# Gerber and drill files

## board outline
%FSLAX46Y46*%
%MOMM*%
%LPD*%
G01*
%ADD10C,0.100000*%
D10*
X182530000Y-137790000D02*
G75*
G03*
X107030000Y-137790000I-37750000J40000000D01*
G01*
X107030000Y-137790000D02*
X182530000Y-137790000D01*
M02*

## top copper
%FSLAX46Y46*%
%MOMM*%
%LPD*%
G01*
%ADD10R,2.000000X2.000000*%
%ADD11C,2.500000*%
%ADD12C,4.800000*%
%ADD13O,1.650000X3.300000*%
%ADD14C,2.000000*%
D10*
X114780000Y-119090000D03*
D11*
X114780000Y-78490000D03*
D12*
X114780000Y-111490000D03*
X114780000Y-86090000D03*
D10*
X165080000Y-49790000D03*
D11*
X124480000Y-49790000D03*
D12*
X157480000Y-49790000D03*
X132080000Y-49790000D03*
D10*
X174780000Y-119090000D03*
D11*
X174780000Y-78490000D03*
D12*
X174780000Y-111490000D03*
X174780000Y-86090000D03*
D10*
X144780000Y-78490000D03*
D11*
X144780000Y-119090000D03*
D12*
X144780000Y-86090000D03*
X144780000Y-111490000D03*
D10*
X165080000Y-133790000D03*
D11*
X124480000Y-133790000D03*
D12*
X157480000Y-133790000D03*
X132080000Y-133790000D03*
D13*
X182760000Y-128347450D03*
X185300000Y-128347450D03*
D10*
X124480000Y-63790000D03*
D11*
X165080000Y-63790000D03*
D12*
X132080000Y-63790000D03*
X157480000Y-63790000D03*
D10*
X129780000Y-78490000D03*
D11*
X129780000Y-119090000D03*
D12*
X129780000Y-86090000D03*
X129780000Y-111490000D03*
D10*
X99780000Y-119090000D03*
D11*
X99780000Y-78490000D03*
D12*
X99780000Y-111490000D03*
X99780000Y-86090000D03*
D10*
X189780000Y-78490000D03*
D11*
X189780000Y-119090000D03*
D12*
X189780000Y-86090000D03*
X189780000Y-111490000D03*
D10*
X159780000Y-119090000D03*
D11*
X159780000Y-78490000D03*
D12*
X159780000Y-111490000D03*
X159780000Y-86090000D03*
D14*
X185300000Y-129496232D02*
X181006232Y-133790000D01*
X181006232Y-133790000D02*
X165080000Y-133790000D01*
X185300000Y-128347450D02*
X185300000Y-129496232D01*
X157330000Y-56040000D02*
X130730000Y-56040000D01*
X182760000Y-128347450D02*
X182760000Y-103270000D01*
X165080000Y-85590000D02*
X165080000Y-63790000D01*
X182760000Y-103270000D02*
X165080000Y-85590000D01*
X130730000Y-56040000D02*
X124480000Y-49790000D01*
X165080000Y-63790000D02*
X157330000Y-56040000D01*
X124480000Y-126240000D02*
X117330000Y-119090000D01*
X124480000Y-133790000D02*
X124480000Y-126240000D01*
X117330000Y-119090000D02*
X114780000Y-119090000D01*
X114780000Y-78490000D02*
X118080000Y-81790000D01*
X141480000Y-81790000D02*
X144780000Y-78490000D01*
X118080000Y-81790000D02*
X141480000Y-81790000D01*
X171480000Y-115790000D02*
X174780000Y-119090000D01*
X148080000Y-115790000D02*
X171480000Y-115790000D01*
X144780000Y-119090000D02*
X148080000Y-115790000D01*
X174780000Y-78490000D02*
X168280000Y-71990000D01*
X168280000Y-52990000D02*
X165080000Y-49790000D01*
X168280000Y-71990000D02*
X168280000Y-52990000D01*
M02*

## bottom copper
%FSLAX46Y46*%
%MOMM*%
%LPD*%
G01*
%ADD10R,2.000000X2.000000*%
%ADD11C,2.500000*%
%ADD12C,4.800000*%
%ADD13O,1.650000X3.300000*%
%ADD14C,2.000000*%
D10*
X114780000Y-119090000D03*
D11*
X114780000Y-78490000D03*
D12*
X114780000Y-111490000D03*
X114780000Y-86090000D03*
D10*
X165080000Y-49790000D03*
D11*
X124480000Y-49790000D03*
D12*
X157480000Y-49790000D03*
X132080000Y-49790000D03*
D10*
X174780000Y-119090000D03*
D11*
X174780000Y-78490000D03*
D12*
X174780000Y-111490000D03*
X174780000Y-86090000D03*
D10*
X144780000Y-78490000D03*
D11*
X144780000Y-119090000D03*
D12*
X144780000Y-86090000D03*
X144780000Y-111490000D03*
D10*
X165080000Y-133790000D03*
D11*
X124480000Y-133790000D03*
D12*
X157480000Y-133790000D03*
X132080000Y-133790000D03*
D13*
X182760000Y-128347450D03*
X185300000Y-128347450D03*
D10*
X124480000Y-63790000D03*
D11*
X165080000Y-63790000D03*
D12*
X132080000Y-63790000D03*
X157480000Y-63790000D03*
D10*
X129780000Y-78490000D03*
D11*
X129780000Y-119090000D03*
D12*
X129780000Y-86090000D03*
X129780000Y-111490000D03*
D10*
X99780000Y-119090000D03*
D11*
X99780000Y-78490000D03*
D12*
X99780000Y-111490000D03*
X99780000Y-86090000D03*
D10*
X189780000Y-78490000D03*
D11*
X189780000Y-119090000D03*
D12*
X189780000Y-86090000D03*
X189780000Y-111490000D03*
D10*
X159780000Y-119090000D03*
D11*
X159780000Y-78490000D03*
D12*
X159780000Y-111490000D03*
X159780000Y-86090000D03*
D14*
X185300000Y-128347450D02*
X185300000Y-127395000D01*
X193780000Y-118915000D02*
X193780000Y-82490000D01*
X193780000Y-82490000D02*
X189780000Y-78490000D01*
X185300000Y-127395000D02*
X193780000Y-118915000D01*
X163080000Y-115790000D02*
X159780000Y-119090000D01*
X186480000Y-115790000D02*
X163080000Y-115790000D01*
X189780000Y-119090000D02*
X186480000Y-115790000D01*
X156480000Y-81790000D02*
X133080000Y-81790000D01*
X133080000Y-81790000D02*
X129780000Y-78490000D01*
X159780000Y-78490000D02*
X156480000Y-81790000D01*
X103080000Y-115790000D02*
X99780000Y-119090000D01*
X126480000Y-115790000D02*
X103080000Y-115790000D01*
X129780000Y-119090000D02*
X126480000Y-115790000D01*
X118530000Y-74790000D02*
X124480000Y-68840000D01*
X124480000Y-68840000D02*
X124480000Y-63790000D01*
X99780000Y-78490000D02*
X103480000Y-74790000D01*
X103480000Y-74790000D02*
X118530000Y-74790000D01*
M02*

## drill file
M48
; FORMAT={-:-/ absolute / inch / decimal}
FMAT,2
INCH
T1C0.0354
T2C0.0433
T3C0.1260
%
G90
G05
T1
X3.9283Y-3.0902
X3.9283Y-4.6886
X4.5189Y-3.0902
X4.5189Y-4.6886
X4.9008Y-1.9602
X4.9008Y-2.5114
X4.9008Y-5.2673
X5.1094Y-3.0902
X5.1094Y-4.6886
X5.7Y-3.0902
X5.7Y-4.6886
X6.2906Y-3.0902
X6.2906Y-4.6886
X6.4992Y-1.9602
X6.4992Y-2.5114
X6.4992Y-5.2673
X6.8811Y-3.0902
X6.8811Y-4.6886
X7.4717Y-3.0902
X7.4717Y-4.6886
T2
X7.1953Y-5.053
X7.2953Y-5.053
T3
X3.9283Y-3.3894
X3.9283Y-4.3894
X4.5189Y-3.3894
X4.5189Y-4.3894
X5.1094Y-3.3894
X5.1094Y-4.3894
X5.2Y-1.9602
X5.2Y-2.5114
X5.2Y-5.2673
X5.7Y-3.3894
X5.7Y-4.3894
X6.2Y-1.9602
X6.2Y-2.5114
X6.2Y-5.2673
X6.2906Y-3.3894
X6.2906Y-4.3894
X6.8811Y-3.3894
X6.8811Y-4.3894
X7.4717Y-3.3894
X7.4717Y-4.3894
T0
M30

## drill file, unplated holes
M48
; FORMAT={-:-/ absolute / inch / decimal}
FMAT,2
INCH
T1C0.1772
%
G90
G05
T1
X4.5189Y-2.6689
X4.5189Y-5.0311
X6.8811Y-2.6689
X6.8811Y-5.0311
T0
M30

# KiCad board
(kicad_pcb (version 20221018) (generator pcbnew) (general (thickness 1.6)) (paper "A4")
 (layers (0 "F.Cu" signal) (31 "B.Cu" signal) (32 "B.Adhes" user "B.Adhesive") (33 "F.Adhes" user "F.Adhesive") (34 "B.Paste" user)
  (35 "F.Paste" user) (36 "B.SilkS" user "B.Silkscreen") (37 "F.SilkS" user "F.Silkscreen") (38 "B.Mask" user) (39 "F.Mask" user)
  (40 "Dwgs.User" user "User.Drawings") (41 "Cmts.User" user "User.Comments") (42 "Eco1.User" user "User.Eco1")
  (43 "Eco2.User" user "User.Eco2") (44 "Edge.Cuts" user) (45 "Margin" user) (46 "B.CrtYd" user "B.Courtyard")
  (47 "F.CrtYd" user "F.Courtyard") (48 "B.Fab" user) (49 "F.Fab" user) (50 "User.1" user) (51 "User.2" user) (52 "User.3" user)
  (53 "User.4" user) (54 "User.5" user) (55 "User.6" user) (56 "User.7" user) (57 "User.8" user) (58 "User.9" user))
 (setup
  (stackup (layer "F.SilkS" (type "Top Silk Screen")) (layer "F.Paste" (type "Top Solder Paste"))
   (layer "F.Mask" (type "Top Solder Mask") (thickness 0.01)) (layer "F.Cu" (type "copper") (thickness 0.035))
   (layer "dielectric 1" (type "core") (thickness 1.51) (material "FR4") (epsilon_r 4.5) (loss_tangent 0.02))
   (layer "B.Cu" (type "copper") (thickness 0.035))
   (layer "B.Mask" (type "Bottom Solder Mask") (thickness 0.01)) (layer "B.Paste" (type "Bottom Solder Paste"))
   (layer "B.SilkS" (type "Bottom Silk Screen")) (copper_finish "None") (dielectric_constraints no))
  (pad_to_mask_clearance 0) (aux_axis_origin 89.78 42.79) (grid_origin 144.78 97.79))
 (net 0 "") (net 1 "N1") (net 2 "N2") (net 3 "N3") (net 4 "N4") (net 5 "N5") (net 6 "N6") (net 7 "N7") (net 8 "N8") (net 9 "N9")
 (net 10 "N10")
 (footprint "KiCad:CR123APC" (layer "F.Cu") (at 114.78 119.09 90)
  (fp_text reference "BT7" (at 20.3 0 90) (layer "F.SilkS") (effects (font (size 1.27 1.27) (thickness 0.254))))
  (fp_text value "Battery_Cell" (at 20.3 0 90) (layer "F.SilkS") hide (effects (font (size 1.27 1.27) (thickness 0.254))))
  (pad "1" thru_hole rect (at 0 0 90) (size 2 2) (drill 0.9) (layers "*.Cu" "*.Mask") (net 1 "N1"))
  (pad "2" thru_hole circle (at 40.6 0 90) (size 2.5 2.5) (drill 0.9) (layers "*.Cu" "*.Mask") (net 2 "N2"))
  (pad "MH1" thru_hole circle (at 7.6 0 90) (size 4.8 4.8) (drill 3.2) (layers "*.Cu" "*.Mask"))
  (pad "MH2" thru_hole circle (at 33 0 90) (size 4.8 4.8) (drill 3.2) (layers "*.Cu" "*.Mask")))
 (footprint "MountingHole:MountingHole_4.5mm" (layer "F.Cu") (at 174.78 127.79)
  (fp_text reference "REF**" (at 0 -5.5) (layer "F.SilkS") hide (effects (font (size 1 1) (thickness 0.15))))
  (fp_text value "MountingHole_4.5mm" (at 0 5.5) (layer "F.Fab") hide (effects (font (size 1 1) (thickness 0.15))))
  (pad "" np_thru_hole circle (at 0 0) (size 4.5 4.5) (drill 4.5) (layers "*.Cu" "*.Mask")))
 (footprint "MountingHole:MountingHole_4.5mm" (layer "F.Cu") (at 174.78 67.79)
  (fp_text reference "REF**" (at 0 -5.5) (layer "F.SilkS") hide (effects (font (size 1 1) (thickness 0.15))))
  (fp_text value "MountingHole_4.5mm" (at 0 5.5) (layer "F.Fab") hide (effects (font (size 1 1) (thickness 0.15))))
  (pad "" np_thru_hole circle (at 0 0) (size 4.5 4.5) (drill 4.5) (layers "*.Cu" "*.Mask")))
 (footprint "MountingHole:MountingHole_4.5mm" (layer "F.Cu") (at 114.78 67.79)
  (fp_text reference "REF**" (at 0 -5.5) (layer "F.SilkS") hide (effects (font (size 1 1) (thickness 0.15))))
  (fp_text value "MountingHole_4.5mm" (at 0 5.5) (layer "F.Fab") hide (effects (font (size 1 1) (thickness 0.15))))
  (pad "" np_thru_hole circle (at 0 0) (size 4.5 4.5) (drill 4.5) (layers "*.Cu" "*.Mask")))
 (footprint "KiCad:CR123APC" (layer "F.Cu") (at 165.08 49.79 180)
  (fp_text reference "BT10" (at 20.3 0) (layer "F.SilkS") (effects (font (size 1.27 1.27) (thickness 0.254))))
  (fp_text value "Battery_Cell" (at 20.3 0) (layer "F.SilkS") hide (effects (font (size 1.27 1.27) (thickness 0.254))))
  (pad "1" thru_hole rect (at 0 0 180) (size 2 2) (drill 0.9) (layers "*.Cu" "*.Mask") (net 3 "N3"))
  (pad "2" thru_hole circle (at 40.6 0 180) (size 2.5 2.5) (drill 0.9) (layers "*.Cu" "*.Mask") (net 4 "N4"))
  (pad "MH1" thru_hole circle (at 7.6 0 180) (size 4.8 4.8) (drill 3.2) (layers "*.Cu" "*.Mask"))
  (pad "MH2" thru_hole circle (at 33 0 180) (size 4.8 4.8) (drill 3.2) (layers "*.Cu" "*.Mask")))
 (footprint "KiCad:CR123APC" (layer "F.Cu") (at 174.78 119.09 90)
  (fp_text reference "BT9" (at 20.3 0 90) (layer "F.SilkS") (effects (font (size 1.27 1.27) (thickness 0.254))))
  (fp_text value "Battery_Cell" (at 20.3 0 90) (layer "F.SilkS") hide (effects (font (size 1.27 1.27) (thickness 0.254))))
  (pad "1" thru_hole rect (at 0 0 90) (size 2 2) (drill 0.9) (layers "*.Cu" "*.Mask") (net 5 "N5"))
  (pad "2" thru_hole circle (at 40.6 0 90) (size 2.5 2.5) (drill 0.9) (layers "*.Cu" "*.Mask") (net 3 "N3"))
  (pad "MH1" thru_hole circle (at 7.6 0 90) (size 4.8 4.8) (drill 3.2) (layers "*.Cu" "*.Mask"))
  (pad "MH2" thru_hole circle (at 33 0 90) (size 4.8 4.8) (drill 3.2) (layers "*.Cu" "*.Mask")))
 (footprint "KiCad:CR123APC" (layer "F.Cu") (at 144.78 78.49 -90)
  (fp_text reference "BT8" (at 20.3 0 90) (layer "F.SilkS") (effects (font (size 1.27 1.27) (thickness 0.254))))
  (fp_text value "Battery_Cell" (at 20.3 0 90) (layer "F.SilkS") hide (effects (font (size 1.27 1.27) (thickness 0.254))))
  (pad "1" thru_hole rect (at 0 0 270) (size 2 2) (drill 0.9) (layers "*.Cu" "*.Mask") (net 2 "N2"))
  (pad "2" thru_hole circle (at 40.6 0 270) (size 2.5 2.5) (drill 0.9) (layers "*.Cu" "*.Mask") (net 5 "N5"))
  (pad "MH1" thru_hole circle (at 7.6 0 270) (size 4.8 4.8) (drill 3.2) (layers "*.Cu" "*.Mask"))
  (pad "MH2" thru_hole circle (at 33 0 270) (size 4.8 4.8) (drill 3.2) (layers "*.Cu" "*.Mask")))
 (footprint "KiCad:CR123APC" (layer "F.Cu") (at 165.08 133.79 180)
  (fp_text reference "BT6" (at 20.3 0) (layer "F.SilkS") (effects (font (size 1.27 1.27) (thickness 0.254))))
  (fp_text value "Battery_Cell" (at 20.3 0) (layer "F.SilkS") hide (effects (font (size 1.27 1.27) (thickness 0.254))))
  (pad "1" thru_hole rect (at 0 0 180) (size 2 2) (drill 0.9) (layers "*.Cu" "*.Mask") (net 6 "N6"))
  (pad "2" thru_hole circle (at 40.6 0 180) (size 2.5 2.5) (drill 0.9) (layers "*.Cu" "*.Mask") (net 1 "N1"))
  (pad "MH1" thru_hole circle (at 7.6 0 180) (size 4.8 4.8) (drill 3.2) (layers "*.Cu" "*.Mask"))
  (pad "MH2" thru_hole circle (at 33 0 180) (size 4.8 4.8) (drill 3.2) (layers "*.Cu" "*.Mask")))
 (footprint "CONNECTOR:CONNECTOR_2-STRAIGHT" (layer "F.Cu") (at 184.03 128.34745)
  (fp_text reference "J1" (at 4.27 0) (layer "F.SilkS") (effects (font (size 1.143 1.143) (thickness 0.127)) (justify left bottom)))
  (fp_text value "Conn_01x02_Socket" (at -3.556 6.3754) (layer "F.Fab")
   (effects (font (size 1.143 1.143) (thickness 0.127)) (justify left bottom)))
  (pad "1" thru_hole oval (at -1.27 0 90) (size 3.3 1.65) (drill 1.1) (layers "*.Cu" "*.Mask") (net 4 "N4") (solder_mask_margin 0.1016)
   (thermal_bridge_angle 45))
  (pad "2" thru_hole oval (at 1.27 0 90) (size 3.3 1.65) (drill 1.1) (layers "*.Cu" "*.Mask") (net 6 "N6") (solder_mask_margin 0.1016)
   (thermal_bridge_angle 45)))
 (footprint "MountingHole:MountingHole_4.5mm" (layer "F.Cu") (at 114.78 127.79)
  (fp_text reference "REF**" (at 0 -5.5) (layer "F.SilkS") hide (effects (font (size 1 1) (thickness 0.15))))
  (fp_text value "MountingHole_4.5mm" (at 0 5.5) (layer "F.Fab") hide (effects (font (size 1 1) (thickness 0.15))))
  (pad "" np_thru_hole circle (at 0 0) (size 4.5 4.5) (drill 4.5) (layers "*.Cu" "*.Mask")))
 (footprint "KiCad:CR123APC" (layer "B.Cu") (at 124.48 63.79)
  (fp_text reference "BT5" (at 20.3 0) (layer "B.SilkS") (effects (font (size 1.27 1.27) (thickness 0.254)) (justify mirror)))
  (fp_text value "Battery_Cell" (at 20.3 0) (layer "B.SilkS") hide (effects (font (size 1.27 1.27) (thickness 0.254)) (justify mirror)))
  (pad "1" thru_hole rect (at 0 0) (size 2 2) (drill 0.9) (layers "*.Cu" "*.Mask") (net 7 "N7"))
  (pad "2" thru_hole circle (at 40.6 0) (size 2.5 2.5) (drill 0.9) (layers "*.Cu" "*.Mask") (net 4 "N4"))
  (pad "MH1" thru_hole circle (at 7.6 0) (size 4.8 4.8) (drill 3.2) (layers "*.Cu" "*.Mask"))
  (pad "MH2" thru_hole circle (at 33 0) (size 4.8 4.8) (drill 3.2) (layers "*.Cu" "*.Mask")))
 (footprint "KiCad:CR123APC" (layer "B.Cu") (at 129.78 78.49 -90)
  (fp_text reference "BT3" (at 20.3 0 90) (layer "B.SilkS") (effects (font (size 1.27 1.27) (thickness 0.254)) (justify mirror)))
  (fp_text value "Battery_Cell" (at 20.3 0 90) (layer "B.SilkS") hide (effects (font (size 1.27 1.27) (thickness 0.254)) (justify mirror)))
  (pad "1" thru_hole rect (at 0 0 270) (size 2 2) (drill 0.9) (layers "*.Cu" "*.Mask") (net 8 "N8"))
  (pad "2" thru_hole circle (at 40.6 0 270) (size 2.5 2.5) (drill 0.9) (layers "*.Cu" "*.Mask") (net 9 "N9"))
  (pad "MH1" thru_hole circle (at 7.6 0 270) (size 4.8 4.8) (drill 3.2) (layers "*.Cu" "*.Mask"))
  (pad "MH2" thru_hole circle (at 33 0 270) (size 4.8 4.8) (drill 3.2) (layers "*.Cu" "*.Mask")))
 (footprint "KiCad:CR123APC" (layer "B.Cu") (at 99.78 119.09 90)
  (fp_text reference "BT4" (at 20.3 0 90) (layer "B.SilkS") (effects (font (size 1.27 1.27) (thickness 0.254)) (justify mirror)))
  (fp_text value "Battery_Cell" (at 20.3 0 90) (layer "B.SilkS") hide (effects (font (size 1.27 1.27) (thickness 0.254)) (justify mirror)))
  (pad "1" thru_hole rect (at 0 0 90) (size 2 2) (drill 0.9) (layers "*.Cu" "*.Mask") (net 9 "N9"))
  (pad "2" thru_hole circle (at 40.6 0 90) (size 2.5 2.5) (drill 0.9) (layers "*.Cu" "*.Mask") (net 7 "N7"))
  (pad "MH1" thru_hole circle (at 7.6 0 90) (size 4.8 4.8) (drill 3.2) (layers "*.Cu" "*.Mask"))
  (pad "MH2" thru_hole circle (at 33 0 90) (size 4.8 4.8) (drill 3.2) (layers "*.Cu" "*.Mask")))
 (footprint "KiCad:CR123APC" (layer "B.Cu") (at 189.78 78.49 -90)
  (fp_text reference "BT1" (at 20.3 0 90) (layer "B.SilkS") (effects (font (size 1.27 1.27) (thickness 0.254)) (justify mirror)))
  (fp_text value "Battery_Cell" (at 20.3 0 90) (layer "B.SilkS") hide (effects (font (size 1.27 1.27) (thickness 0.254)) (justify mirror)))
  (pad "1" thru_hole rect (at 0 0 270) (size 2 2) (drill 0.9) (layers "*.Cu" "*.Mask") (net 6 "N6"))
  (pad "2" thru_hole circle (at 40.6 0 270) (size 2.5 2.5) (drill 0.9) (layers "*.Cu" "*.Mask") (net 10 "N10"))
  (pad "MH1" thru_hole circle (at 7.6 0 270) (size 4.8 4.8) (drill 3.2) (layers "*.Cu" "*.Mask"))
  (pad "MH2" thru_hole circle (at 33 0 270) (size 4.8 4.8) (drill 3.2) (layers "*.Cu" "*.Mask")))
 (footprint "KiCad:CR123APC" (layer "B.Cu") (at 159.78 119.09 90)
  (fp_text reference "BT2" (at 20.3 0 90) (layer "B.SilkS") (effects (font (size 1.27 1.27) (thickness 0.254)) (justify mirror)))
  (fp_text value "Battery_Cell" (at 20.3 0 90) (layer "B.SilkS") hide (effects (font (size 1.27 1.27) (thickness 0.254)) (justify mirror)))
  (pad "1" thru_hole rect (at 0 0 90) (size 2 2) (drill 0.9) (layers "*.Cu" "*.Mask") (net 10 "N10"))
  (pad "2" thru_hole circle (at 40.6 0 90) (size 2.5 2.5) (drill 0.9) (layers "*.Cu" "*.Mask") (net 8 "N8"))
  (pad "MH1" thru_hole circle (at 7.6 0 90) (size 4.8 4.8) (drill 3.2) (layers "*.Cu" "*.Mask"))
  (pad "MH2" thru_hole circle (at 33 0 90) (size 4.8 4.8) (drill 3.2) (layers "*.Cu" "*.Mask")))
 (gr_arc (start 107.03 137.79) (mid 144.78 42.789432) (end 182.53 137.79) (stroke (width 0.1) (type default)) (layer "Edge.Cuts"))
 (gr_line (start 107.03 137.79) (end 182.53 137.79) (stroke (width 0.1) (type default)) (layer "Edge.Cuts"))
 (segment (start 185.3 129.496232) (end 181.006232 133.79) (width 2) (layer "F.Cu") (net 6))
 (segment (start 181.006232 133.79) (end 165.08 133.79) (width 2) (layer "F.Cu") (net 6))
 (segment (start 185.3 128.34745) (end 185.3 129.496232) (width 2) (layer "F.Cu") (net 6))
 (segment (start 185.3 128.34745) (end 185.3 127.395) (width 2) (layer "B.Cu") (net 6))
 (segment (start 193.78 118.915) (end 193.78 82.49) (width 2) (layer "B.Cu") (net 6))
 (segment (start 193.78 82.49) (end 189.78 78.49) (width 2) (layer "B.Cu") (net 6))
 (segment (start 185.3 127.395) (end 193.78 118.915) (width 2) (layer "B.Cu") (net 6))
 (segment (start 163.08 115.79) (end 159.78 119.09) (width 2) (layer "B.Cu") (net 10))
 (segment (start 186.48 115.79) (end 163.08 115.79) (width 2) (layer "B.Cu") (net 10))
 (segment (start 189.78 119.09) (end 186.48 115.79) (width 2) (layer "B.Cu") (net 10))
 (segment (start 156.48 81.79) (end 133.08 81.79) (width 2) (layer "B.Cu") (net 8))
 (segment (start 133.08 81.79) (end 129.78 78.49) (width 2) (layer "B.Cu") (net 8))
 (segment (start 159.78 78.49) (end 156.48 81.79) (width 2) (layer "B.Cu") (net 8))
 (segment (start 103.08 115.79) (end 99.78 119.09) (width 2) (layer "B.Cu") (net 9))
 (segment (start 126.48 115.79) (end 103.08 115.79) (width 2) (layer "B.Cu") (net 9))
 (segment (start 129.78 119.09) (end 126.48 115.79) (width 2) (layer "B.Cu") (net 9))
 (segment (start 118.53 74.79) (end 124.48 68.84) (width 2) (layer "B.Cu") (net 7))
 (segment (start 124.48 68.84) (end 124.48 63.79) (width 2) (layer "B.Cu") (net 7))
 (segment (start 99.78 78.49) (end 103.48 74.79) (width 2) (layer "B.Cu") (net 7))
 (segment (start 103.48 74.79) (end 118.53 74.79) (width 2) (layer "B.Cu") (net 7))
 (segment (start 157.33 56.04) (end 130.73 56.04) (width 2) (layer "F.Cu") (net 4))
 (segment (start 182.76 128.34745) (end 182.76 103.27) (width 2) (layer "F.Cu") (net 4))
 (segment (start 165.08 85.59) (end 165.08 63.79) (width 2) (layer "F.Cu") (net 4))
 (segment (start 182.76 103.27) (end 165.08 85.59) (width 2) (layer "F.Cu") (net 4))
 (segment (start 130.73 56.04) (end 124.48 49.79) (width 2) (layer "F.Cu") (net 4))
 (segment (start 165.08 63.79) (end 157.33 56.04) (width 2) (layer "F.Cu") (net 4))
 (segment (start 124.48 126.24) (end 117.33 119.09) (width 2) (layer "F.Cu") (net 1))
 (segment (start 124.48 133.79) (end 124.48 126.24) (width 2) (layer "F.Cu") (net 1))
 (segment (start 117.33 119.09) (end 114.78 119.09) (width 2) (layer "F.Cu") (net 1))
 (segment (start 114.78 78.49) (end 118.08 81.79) (width 2) (layer "F.Cu") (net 2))
 (segment (start 141.48 81.79) (end 144.78 78.49) (width 2) (layer "F.Cu") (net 2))
 (segment (start 118.08 81.79) (end 141.48 81.79) (width 2) (layer "F.Cu") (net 2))
 (segment (start 171.48 115.79) (end 174.78 119.09) (width 2) (layer "F.Cu") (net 5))
 (segment (start 148.08 115.79) (end 171.48 115.79) (width 2) (layer "F.Cu") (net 5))
 (segment (start 144.78 119.09) (end 148.08 115.79) (width 2) (layer "F.Cu") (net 5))
 (segment (start 174.78 78.49) (end 168.28 71.99) (width 2) (layer "F.Cu") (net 3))
 (segment (start 168.28 52.99) (end 165.08 49.79) (width 2) (layer "F.Cu") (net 3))
 (segment (start 168.28 71.99) (end 168.28 52.99) (width 2) (layer "F.Cu") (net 3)))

